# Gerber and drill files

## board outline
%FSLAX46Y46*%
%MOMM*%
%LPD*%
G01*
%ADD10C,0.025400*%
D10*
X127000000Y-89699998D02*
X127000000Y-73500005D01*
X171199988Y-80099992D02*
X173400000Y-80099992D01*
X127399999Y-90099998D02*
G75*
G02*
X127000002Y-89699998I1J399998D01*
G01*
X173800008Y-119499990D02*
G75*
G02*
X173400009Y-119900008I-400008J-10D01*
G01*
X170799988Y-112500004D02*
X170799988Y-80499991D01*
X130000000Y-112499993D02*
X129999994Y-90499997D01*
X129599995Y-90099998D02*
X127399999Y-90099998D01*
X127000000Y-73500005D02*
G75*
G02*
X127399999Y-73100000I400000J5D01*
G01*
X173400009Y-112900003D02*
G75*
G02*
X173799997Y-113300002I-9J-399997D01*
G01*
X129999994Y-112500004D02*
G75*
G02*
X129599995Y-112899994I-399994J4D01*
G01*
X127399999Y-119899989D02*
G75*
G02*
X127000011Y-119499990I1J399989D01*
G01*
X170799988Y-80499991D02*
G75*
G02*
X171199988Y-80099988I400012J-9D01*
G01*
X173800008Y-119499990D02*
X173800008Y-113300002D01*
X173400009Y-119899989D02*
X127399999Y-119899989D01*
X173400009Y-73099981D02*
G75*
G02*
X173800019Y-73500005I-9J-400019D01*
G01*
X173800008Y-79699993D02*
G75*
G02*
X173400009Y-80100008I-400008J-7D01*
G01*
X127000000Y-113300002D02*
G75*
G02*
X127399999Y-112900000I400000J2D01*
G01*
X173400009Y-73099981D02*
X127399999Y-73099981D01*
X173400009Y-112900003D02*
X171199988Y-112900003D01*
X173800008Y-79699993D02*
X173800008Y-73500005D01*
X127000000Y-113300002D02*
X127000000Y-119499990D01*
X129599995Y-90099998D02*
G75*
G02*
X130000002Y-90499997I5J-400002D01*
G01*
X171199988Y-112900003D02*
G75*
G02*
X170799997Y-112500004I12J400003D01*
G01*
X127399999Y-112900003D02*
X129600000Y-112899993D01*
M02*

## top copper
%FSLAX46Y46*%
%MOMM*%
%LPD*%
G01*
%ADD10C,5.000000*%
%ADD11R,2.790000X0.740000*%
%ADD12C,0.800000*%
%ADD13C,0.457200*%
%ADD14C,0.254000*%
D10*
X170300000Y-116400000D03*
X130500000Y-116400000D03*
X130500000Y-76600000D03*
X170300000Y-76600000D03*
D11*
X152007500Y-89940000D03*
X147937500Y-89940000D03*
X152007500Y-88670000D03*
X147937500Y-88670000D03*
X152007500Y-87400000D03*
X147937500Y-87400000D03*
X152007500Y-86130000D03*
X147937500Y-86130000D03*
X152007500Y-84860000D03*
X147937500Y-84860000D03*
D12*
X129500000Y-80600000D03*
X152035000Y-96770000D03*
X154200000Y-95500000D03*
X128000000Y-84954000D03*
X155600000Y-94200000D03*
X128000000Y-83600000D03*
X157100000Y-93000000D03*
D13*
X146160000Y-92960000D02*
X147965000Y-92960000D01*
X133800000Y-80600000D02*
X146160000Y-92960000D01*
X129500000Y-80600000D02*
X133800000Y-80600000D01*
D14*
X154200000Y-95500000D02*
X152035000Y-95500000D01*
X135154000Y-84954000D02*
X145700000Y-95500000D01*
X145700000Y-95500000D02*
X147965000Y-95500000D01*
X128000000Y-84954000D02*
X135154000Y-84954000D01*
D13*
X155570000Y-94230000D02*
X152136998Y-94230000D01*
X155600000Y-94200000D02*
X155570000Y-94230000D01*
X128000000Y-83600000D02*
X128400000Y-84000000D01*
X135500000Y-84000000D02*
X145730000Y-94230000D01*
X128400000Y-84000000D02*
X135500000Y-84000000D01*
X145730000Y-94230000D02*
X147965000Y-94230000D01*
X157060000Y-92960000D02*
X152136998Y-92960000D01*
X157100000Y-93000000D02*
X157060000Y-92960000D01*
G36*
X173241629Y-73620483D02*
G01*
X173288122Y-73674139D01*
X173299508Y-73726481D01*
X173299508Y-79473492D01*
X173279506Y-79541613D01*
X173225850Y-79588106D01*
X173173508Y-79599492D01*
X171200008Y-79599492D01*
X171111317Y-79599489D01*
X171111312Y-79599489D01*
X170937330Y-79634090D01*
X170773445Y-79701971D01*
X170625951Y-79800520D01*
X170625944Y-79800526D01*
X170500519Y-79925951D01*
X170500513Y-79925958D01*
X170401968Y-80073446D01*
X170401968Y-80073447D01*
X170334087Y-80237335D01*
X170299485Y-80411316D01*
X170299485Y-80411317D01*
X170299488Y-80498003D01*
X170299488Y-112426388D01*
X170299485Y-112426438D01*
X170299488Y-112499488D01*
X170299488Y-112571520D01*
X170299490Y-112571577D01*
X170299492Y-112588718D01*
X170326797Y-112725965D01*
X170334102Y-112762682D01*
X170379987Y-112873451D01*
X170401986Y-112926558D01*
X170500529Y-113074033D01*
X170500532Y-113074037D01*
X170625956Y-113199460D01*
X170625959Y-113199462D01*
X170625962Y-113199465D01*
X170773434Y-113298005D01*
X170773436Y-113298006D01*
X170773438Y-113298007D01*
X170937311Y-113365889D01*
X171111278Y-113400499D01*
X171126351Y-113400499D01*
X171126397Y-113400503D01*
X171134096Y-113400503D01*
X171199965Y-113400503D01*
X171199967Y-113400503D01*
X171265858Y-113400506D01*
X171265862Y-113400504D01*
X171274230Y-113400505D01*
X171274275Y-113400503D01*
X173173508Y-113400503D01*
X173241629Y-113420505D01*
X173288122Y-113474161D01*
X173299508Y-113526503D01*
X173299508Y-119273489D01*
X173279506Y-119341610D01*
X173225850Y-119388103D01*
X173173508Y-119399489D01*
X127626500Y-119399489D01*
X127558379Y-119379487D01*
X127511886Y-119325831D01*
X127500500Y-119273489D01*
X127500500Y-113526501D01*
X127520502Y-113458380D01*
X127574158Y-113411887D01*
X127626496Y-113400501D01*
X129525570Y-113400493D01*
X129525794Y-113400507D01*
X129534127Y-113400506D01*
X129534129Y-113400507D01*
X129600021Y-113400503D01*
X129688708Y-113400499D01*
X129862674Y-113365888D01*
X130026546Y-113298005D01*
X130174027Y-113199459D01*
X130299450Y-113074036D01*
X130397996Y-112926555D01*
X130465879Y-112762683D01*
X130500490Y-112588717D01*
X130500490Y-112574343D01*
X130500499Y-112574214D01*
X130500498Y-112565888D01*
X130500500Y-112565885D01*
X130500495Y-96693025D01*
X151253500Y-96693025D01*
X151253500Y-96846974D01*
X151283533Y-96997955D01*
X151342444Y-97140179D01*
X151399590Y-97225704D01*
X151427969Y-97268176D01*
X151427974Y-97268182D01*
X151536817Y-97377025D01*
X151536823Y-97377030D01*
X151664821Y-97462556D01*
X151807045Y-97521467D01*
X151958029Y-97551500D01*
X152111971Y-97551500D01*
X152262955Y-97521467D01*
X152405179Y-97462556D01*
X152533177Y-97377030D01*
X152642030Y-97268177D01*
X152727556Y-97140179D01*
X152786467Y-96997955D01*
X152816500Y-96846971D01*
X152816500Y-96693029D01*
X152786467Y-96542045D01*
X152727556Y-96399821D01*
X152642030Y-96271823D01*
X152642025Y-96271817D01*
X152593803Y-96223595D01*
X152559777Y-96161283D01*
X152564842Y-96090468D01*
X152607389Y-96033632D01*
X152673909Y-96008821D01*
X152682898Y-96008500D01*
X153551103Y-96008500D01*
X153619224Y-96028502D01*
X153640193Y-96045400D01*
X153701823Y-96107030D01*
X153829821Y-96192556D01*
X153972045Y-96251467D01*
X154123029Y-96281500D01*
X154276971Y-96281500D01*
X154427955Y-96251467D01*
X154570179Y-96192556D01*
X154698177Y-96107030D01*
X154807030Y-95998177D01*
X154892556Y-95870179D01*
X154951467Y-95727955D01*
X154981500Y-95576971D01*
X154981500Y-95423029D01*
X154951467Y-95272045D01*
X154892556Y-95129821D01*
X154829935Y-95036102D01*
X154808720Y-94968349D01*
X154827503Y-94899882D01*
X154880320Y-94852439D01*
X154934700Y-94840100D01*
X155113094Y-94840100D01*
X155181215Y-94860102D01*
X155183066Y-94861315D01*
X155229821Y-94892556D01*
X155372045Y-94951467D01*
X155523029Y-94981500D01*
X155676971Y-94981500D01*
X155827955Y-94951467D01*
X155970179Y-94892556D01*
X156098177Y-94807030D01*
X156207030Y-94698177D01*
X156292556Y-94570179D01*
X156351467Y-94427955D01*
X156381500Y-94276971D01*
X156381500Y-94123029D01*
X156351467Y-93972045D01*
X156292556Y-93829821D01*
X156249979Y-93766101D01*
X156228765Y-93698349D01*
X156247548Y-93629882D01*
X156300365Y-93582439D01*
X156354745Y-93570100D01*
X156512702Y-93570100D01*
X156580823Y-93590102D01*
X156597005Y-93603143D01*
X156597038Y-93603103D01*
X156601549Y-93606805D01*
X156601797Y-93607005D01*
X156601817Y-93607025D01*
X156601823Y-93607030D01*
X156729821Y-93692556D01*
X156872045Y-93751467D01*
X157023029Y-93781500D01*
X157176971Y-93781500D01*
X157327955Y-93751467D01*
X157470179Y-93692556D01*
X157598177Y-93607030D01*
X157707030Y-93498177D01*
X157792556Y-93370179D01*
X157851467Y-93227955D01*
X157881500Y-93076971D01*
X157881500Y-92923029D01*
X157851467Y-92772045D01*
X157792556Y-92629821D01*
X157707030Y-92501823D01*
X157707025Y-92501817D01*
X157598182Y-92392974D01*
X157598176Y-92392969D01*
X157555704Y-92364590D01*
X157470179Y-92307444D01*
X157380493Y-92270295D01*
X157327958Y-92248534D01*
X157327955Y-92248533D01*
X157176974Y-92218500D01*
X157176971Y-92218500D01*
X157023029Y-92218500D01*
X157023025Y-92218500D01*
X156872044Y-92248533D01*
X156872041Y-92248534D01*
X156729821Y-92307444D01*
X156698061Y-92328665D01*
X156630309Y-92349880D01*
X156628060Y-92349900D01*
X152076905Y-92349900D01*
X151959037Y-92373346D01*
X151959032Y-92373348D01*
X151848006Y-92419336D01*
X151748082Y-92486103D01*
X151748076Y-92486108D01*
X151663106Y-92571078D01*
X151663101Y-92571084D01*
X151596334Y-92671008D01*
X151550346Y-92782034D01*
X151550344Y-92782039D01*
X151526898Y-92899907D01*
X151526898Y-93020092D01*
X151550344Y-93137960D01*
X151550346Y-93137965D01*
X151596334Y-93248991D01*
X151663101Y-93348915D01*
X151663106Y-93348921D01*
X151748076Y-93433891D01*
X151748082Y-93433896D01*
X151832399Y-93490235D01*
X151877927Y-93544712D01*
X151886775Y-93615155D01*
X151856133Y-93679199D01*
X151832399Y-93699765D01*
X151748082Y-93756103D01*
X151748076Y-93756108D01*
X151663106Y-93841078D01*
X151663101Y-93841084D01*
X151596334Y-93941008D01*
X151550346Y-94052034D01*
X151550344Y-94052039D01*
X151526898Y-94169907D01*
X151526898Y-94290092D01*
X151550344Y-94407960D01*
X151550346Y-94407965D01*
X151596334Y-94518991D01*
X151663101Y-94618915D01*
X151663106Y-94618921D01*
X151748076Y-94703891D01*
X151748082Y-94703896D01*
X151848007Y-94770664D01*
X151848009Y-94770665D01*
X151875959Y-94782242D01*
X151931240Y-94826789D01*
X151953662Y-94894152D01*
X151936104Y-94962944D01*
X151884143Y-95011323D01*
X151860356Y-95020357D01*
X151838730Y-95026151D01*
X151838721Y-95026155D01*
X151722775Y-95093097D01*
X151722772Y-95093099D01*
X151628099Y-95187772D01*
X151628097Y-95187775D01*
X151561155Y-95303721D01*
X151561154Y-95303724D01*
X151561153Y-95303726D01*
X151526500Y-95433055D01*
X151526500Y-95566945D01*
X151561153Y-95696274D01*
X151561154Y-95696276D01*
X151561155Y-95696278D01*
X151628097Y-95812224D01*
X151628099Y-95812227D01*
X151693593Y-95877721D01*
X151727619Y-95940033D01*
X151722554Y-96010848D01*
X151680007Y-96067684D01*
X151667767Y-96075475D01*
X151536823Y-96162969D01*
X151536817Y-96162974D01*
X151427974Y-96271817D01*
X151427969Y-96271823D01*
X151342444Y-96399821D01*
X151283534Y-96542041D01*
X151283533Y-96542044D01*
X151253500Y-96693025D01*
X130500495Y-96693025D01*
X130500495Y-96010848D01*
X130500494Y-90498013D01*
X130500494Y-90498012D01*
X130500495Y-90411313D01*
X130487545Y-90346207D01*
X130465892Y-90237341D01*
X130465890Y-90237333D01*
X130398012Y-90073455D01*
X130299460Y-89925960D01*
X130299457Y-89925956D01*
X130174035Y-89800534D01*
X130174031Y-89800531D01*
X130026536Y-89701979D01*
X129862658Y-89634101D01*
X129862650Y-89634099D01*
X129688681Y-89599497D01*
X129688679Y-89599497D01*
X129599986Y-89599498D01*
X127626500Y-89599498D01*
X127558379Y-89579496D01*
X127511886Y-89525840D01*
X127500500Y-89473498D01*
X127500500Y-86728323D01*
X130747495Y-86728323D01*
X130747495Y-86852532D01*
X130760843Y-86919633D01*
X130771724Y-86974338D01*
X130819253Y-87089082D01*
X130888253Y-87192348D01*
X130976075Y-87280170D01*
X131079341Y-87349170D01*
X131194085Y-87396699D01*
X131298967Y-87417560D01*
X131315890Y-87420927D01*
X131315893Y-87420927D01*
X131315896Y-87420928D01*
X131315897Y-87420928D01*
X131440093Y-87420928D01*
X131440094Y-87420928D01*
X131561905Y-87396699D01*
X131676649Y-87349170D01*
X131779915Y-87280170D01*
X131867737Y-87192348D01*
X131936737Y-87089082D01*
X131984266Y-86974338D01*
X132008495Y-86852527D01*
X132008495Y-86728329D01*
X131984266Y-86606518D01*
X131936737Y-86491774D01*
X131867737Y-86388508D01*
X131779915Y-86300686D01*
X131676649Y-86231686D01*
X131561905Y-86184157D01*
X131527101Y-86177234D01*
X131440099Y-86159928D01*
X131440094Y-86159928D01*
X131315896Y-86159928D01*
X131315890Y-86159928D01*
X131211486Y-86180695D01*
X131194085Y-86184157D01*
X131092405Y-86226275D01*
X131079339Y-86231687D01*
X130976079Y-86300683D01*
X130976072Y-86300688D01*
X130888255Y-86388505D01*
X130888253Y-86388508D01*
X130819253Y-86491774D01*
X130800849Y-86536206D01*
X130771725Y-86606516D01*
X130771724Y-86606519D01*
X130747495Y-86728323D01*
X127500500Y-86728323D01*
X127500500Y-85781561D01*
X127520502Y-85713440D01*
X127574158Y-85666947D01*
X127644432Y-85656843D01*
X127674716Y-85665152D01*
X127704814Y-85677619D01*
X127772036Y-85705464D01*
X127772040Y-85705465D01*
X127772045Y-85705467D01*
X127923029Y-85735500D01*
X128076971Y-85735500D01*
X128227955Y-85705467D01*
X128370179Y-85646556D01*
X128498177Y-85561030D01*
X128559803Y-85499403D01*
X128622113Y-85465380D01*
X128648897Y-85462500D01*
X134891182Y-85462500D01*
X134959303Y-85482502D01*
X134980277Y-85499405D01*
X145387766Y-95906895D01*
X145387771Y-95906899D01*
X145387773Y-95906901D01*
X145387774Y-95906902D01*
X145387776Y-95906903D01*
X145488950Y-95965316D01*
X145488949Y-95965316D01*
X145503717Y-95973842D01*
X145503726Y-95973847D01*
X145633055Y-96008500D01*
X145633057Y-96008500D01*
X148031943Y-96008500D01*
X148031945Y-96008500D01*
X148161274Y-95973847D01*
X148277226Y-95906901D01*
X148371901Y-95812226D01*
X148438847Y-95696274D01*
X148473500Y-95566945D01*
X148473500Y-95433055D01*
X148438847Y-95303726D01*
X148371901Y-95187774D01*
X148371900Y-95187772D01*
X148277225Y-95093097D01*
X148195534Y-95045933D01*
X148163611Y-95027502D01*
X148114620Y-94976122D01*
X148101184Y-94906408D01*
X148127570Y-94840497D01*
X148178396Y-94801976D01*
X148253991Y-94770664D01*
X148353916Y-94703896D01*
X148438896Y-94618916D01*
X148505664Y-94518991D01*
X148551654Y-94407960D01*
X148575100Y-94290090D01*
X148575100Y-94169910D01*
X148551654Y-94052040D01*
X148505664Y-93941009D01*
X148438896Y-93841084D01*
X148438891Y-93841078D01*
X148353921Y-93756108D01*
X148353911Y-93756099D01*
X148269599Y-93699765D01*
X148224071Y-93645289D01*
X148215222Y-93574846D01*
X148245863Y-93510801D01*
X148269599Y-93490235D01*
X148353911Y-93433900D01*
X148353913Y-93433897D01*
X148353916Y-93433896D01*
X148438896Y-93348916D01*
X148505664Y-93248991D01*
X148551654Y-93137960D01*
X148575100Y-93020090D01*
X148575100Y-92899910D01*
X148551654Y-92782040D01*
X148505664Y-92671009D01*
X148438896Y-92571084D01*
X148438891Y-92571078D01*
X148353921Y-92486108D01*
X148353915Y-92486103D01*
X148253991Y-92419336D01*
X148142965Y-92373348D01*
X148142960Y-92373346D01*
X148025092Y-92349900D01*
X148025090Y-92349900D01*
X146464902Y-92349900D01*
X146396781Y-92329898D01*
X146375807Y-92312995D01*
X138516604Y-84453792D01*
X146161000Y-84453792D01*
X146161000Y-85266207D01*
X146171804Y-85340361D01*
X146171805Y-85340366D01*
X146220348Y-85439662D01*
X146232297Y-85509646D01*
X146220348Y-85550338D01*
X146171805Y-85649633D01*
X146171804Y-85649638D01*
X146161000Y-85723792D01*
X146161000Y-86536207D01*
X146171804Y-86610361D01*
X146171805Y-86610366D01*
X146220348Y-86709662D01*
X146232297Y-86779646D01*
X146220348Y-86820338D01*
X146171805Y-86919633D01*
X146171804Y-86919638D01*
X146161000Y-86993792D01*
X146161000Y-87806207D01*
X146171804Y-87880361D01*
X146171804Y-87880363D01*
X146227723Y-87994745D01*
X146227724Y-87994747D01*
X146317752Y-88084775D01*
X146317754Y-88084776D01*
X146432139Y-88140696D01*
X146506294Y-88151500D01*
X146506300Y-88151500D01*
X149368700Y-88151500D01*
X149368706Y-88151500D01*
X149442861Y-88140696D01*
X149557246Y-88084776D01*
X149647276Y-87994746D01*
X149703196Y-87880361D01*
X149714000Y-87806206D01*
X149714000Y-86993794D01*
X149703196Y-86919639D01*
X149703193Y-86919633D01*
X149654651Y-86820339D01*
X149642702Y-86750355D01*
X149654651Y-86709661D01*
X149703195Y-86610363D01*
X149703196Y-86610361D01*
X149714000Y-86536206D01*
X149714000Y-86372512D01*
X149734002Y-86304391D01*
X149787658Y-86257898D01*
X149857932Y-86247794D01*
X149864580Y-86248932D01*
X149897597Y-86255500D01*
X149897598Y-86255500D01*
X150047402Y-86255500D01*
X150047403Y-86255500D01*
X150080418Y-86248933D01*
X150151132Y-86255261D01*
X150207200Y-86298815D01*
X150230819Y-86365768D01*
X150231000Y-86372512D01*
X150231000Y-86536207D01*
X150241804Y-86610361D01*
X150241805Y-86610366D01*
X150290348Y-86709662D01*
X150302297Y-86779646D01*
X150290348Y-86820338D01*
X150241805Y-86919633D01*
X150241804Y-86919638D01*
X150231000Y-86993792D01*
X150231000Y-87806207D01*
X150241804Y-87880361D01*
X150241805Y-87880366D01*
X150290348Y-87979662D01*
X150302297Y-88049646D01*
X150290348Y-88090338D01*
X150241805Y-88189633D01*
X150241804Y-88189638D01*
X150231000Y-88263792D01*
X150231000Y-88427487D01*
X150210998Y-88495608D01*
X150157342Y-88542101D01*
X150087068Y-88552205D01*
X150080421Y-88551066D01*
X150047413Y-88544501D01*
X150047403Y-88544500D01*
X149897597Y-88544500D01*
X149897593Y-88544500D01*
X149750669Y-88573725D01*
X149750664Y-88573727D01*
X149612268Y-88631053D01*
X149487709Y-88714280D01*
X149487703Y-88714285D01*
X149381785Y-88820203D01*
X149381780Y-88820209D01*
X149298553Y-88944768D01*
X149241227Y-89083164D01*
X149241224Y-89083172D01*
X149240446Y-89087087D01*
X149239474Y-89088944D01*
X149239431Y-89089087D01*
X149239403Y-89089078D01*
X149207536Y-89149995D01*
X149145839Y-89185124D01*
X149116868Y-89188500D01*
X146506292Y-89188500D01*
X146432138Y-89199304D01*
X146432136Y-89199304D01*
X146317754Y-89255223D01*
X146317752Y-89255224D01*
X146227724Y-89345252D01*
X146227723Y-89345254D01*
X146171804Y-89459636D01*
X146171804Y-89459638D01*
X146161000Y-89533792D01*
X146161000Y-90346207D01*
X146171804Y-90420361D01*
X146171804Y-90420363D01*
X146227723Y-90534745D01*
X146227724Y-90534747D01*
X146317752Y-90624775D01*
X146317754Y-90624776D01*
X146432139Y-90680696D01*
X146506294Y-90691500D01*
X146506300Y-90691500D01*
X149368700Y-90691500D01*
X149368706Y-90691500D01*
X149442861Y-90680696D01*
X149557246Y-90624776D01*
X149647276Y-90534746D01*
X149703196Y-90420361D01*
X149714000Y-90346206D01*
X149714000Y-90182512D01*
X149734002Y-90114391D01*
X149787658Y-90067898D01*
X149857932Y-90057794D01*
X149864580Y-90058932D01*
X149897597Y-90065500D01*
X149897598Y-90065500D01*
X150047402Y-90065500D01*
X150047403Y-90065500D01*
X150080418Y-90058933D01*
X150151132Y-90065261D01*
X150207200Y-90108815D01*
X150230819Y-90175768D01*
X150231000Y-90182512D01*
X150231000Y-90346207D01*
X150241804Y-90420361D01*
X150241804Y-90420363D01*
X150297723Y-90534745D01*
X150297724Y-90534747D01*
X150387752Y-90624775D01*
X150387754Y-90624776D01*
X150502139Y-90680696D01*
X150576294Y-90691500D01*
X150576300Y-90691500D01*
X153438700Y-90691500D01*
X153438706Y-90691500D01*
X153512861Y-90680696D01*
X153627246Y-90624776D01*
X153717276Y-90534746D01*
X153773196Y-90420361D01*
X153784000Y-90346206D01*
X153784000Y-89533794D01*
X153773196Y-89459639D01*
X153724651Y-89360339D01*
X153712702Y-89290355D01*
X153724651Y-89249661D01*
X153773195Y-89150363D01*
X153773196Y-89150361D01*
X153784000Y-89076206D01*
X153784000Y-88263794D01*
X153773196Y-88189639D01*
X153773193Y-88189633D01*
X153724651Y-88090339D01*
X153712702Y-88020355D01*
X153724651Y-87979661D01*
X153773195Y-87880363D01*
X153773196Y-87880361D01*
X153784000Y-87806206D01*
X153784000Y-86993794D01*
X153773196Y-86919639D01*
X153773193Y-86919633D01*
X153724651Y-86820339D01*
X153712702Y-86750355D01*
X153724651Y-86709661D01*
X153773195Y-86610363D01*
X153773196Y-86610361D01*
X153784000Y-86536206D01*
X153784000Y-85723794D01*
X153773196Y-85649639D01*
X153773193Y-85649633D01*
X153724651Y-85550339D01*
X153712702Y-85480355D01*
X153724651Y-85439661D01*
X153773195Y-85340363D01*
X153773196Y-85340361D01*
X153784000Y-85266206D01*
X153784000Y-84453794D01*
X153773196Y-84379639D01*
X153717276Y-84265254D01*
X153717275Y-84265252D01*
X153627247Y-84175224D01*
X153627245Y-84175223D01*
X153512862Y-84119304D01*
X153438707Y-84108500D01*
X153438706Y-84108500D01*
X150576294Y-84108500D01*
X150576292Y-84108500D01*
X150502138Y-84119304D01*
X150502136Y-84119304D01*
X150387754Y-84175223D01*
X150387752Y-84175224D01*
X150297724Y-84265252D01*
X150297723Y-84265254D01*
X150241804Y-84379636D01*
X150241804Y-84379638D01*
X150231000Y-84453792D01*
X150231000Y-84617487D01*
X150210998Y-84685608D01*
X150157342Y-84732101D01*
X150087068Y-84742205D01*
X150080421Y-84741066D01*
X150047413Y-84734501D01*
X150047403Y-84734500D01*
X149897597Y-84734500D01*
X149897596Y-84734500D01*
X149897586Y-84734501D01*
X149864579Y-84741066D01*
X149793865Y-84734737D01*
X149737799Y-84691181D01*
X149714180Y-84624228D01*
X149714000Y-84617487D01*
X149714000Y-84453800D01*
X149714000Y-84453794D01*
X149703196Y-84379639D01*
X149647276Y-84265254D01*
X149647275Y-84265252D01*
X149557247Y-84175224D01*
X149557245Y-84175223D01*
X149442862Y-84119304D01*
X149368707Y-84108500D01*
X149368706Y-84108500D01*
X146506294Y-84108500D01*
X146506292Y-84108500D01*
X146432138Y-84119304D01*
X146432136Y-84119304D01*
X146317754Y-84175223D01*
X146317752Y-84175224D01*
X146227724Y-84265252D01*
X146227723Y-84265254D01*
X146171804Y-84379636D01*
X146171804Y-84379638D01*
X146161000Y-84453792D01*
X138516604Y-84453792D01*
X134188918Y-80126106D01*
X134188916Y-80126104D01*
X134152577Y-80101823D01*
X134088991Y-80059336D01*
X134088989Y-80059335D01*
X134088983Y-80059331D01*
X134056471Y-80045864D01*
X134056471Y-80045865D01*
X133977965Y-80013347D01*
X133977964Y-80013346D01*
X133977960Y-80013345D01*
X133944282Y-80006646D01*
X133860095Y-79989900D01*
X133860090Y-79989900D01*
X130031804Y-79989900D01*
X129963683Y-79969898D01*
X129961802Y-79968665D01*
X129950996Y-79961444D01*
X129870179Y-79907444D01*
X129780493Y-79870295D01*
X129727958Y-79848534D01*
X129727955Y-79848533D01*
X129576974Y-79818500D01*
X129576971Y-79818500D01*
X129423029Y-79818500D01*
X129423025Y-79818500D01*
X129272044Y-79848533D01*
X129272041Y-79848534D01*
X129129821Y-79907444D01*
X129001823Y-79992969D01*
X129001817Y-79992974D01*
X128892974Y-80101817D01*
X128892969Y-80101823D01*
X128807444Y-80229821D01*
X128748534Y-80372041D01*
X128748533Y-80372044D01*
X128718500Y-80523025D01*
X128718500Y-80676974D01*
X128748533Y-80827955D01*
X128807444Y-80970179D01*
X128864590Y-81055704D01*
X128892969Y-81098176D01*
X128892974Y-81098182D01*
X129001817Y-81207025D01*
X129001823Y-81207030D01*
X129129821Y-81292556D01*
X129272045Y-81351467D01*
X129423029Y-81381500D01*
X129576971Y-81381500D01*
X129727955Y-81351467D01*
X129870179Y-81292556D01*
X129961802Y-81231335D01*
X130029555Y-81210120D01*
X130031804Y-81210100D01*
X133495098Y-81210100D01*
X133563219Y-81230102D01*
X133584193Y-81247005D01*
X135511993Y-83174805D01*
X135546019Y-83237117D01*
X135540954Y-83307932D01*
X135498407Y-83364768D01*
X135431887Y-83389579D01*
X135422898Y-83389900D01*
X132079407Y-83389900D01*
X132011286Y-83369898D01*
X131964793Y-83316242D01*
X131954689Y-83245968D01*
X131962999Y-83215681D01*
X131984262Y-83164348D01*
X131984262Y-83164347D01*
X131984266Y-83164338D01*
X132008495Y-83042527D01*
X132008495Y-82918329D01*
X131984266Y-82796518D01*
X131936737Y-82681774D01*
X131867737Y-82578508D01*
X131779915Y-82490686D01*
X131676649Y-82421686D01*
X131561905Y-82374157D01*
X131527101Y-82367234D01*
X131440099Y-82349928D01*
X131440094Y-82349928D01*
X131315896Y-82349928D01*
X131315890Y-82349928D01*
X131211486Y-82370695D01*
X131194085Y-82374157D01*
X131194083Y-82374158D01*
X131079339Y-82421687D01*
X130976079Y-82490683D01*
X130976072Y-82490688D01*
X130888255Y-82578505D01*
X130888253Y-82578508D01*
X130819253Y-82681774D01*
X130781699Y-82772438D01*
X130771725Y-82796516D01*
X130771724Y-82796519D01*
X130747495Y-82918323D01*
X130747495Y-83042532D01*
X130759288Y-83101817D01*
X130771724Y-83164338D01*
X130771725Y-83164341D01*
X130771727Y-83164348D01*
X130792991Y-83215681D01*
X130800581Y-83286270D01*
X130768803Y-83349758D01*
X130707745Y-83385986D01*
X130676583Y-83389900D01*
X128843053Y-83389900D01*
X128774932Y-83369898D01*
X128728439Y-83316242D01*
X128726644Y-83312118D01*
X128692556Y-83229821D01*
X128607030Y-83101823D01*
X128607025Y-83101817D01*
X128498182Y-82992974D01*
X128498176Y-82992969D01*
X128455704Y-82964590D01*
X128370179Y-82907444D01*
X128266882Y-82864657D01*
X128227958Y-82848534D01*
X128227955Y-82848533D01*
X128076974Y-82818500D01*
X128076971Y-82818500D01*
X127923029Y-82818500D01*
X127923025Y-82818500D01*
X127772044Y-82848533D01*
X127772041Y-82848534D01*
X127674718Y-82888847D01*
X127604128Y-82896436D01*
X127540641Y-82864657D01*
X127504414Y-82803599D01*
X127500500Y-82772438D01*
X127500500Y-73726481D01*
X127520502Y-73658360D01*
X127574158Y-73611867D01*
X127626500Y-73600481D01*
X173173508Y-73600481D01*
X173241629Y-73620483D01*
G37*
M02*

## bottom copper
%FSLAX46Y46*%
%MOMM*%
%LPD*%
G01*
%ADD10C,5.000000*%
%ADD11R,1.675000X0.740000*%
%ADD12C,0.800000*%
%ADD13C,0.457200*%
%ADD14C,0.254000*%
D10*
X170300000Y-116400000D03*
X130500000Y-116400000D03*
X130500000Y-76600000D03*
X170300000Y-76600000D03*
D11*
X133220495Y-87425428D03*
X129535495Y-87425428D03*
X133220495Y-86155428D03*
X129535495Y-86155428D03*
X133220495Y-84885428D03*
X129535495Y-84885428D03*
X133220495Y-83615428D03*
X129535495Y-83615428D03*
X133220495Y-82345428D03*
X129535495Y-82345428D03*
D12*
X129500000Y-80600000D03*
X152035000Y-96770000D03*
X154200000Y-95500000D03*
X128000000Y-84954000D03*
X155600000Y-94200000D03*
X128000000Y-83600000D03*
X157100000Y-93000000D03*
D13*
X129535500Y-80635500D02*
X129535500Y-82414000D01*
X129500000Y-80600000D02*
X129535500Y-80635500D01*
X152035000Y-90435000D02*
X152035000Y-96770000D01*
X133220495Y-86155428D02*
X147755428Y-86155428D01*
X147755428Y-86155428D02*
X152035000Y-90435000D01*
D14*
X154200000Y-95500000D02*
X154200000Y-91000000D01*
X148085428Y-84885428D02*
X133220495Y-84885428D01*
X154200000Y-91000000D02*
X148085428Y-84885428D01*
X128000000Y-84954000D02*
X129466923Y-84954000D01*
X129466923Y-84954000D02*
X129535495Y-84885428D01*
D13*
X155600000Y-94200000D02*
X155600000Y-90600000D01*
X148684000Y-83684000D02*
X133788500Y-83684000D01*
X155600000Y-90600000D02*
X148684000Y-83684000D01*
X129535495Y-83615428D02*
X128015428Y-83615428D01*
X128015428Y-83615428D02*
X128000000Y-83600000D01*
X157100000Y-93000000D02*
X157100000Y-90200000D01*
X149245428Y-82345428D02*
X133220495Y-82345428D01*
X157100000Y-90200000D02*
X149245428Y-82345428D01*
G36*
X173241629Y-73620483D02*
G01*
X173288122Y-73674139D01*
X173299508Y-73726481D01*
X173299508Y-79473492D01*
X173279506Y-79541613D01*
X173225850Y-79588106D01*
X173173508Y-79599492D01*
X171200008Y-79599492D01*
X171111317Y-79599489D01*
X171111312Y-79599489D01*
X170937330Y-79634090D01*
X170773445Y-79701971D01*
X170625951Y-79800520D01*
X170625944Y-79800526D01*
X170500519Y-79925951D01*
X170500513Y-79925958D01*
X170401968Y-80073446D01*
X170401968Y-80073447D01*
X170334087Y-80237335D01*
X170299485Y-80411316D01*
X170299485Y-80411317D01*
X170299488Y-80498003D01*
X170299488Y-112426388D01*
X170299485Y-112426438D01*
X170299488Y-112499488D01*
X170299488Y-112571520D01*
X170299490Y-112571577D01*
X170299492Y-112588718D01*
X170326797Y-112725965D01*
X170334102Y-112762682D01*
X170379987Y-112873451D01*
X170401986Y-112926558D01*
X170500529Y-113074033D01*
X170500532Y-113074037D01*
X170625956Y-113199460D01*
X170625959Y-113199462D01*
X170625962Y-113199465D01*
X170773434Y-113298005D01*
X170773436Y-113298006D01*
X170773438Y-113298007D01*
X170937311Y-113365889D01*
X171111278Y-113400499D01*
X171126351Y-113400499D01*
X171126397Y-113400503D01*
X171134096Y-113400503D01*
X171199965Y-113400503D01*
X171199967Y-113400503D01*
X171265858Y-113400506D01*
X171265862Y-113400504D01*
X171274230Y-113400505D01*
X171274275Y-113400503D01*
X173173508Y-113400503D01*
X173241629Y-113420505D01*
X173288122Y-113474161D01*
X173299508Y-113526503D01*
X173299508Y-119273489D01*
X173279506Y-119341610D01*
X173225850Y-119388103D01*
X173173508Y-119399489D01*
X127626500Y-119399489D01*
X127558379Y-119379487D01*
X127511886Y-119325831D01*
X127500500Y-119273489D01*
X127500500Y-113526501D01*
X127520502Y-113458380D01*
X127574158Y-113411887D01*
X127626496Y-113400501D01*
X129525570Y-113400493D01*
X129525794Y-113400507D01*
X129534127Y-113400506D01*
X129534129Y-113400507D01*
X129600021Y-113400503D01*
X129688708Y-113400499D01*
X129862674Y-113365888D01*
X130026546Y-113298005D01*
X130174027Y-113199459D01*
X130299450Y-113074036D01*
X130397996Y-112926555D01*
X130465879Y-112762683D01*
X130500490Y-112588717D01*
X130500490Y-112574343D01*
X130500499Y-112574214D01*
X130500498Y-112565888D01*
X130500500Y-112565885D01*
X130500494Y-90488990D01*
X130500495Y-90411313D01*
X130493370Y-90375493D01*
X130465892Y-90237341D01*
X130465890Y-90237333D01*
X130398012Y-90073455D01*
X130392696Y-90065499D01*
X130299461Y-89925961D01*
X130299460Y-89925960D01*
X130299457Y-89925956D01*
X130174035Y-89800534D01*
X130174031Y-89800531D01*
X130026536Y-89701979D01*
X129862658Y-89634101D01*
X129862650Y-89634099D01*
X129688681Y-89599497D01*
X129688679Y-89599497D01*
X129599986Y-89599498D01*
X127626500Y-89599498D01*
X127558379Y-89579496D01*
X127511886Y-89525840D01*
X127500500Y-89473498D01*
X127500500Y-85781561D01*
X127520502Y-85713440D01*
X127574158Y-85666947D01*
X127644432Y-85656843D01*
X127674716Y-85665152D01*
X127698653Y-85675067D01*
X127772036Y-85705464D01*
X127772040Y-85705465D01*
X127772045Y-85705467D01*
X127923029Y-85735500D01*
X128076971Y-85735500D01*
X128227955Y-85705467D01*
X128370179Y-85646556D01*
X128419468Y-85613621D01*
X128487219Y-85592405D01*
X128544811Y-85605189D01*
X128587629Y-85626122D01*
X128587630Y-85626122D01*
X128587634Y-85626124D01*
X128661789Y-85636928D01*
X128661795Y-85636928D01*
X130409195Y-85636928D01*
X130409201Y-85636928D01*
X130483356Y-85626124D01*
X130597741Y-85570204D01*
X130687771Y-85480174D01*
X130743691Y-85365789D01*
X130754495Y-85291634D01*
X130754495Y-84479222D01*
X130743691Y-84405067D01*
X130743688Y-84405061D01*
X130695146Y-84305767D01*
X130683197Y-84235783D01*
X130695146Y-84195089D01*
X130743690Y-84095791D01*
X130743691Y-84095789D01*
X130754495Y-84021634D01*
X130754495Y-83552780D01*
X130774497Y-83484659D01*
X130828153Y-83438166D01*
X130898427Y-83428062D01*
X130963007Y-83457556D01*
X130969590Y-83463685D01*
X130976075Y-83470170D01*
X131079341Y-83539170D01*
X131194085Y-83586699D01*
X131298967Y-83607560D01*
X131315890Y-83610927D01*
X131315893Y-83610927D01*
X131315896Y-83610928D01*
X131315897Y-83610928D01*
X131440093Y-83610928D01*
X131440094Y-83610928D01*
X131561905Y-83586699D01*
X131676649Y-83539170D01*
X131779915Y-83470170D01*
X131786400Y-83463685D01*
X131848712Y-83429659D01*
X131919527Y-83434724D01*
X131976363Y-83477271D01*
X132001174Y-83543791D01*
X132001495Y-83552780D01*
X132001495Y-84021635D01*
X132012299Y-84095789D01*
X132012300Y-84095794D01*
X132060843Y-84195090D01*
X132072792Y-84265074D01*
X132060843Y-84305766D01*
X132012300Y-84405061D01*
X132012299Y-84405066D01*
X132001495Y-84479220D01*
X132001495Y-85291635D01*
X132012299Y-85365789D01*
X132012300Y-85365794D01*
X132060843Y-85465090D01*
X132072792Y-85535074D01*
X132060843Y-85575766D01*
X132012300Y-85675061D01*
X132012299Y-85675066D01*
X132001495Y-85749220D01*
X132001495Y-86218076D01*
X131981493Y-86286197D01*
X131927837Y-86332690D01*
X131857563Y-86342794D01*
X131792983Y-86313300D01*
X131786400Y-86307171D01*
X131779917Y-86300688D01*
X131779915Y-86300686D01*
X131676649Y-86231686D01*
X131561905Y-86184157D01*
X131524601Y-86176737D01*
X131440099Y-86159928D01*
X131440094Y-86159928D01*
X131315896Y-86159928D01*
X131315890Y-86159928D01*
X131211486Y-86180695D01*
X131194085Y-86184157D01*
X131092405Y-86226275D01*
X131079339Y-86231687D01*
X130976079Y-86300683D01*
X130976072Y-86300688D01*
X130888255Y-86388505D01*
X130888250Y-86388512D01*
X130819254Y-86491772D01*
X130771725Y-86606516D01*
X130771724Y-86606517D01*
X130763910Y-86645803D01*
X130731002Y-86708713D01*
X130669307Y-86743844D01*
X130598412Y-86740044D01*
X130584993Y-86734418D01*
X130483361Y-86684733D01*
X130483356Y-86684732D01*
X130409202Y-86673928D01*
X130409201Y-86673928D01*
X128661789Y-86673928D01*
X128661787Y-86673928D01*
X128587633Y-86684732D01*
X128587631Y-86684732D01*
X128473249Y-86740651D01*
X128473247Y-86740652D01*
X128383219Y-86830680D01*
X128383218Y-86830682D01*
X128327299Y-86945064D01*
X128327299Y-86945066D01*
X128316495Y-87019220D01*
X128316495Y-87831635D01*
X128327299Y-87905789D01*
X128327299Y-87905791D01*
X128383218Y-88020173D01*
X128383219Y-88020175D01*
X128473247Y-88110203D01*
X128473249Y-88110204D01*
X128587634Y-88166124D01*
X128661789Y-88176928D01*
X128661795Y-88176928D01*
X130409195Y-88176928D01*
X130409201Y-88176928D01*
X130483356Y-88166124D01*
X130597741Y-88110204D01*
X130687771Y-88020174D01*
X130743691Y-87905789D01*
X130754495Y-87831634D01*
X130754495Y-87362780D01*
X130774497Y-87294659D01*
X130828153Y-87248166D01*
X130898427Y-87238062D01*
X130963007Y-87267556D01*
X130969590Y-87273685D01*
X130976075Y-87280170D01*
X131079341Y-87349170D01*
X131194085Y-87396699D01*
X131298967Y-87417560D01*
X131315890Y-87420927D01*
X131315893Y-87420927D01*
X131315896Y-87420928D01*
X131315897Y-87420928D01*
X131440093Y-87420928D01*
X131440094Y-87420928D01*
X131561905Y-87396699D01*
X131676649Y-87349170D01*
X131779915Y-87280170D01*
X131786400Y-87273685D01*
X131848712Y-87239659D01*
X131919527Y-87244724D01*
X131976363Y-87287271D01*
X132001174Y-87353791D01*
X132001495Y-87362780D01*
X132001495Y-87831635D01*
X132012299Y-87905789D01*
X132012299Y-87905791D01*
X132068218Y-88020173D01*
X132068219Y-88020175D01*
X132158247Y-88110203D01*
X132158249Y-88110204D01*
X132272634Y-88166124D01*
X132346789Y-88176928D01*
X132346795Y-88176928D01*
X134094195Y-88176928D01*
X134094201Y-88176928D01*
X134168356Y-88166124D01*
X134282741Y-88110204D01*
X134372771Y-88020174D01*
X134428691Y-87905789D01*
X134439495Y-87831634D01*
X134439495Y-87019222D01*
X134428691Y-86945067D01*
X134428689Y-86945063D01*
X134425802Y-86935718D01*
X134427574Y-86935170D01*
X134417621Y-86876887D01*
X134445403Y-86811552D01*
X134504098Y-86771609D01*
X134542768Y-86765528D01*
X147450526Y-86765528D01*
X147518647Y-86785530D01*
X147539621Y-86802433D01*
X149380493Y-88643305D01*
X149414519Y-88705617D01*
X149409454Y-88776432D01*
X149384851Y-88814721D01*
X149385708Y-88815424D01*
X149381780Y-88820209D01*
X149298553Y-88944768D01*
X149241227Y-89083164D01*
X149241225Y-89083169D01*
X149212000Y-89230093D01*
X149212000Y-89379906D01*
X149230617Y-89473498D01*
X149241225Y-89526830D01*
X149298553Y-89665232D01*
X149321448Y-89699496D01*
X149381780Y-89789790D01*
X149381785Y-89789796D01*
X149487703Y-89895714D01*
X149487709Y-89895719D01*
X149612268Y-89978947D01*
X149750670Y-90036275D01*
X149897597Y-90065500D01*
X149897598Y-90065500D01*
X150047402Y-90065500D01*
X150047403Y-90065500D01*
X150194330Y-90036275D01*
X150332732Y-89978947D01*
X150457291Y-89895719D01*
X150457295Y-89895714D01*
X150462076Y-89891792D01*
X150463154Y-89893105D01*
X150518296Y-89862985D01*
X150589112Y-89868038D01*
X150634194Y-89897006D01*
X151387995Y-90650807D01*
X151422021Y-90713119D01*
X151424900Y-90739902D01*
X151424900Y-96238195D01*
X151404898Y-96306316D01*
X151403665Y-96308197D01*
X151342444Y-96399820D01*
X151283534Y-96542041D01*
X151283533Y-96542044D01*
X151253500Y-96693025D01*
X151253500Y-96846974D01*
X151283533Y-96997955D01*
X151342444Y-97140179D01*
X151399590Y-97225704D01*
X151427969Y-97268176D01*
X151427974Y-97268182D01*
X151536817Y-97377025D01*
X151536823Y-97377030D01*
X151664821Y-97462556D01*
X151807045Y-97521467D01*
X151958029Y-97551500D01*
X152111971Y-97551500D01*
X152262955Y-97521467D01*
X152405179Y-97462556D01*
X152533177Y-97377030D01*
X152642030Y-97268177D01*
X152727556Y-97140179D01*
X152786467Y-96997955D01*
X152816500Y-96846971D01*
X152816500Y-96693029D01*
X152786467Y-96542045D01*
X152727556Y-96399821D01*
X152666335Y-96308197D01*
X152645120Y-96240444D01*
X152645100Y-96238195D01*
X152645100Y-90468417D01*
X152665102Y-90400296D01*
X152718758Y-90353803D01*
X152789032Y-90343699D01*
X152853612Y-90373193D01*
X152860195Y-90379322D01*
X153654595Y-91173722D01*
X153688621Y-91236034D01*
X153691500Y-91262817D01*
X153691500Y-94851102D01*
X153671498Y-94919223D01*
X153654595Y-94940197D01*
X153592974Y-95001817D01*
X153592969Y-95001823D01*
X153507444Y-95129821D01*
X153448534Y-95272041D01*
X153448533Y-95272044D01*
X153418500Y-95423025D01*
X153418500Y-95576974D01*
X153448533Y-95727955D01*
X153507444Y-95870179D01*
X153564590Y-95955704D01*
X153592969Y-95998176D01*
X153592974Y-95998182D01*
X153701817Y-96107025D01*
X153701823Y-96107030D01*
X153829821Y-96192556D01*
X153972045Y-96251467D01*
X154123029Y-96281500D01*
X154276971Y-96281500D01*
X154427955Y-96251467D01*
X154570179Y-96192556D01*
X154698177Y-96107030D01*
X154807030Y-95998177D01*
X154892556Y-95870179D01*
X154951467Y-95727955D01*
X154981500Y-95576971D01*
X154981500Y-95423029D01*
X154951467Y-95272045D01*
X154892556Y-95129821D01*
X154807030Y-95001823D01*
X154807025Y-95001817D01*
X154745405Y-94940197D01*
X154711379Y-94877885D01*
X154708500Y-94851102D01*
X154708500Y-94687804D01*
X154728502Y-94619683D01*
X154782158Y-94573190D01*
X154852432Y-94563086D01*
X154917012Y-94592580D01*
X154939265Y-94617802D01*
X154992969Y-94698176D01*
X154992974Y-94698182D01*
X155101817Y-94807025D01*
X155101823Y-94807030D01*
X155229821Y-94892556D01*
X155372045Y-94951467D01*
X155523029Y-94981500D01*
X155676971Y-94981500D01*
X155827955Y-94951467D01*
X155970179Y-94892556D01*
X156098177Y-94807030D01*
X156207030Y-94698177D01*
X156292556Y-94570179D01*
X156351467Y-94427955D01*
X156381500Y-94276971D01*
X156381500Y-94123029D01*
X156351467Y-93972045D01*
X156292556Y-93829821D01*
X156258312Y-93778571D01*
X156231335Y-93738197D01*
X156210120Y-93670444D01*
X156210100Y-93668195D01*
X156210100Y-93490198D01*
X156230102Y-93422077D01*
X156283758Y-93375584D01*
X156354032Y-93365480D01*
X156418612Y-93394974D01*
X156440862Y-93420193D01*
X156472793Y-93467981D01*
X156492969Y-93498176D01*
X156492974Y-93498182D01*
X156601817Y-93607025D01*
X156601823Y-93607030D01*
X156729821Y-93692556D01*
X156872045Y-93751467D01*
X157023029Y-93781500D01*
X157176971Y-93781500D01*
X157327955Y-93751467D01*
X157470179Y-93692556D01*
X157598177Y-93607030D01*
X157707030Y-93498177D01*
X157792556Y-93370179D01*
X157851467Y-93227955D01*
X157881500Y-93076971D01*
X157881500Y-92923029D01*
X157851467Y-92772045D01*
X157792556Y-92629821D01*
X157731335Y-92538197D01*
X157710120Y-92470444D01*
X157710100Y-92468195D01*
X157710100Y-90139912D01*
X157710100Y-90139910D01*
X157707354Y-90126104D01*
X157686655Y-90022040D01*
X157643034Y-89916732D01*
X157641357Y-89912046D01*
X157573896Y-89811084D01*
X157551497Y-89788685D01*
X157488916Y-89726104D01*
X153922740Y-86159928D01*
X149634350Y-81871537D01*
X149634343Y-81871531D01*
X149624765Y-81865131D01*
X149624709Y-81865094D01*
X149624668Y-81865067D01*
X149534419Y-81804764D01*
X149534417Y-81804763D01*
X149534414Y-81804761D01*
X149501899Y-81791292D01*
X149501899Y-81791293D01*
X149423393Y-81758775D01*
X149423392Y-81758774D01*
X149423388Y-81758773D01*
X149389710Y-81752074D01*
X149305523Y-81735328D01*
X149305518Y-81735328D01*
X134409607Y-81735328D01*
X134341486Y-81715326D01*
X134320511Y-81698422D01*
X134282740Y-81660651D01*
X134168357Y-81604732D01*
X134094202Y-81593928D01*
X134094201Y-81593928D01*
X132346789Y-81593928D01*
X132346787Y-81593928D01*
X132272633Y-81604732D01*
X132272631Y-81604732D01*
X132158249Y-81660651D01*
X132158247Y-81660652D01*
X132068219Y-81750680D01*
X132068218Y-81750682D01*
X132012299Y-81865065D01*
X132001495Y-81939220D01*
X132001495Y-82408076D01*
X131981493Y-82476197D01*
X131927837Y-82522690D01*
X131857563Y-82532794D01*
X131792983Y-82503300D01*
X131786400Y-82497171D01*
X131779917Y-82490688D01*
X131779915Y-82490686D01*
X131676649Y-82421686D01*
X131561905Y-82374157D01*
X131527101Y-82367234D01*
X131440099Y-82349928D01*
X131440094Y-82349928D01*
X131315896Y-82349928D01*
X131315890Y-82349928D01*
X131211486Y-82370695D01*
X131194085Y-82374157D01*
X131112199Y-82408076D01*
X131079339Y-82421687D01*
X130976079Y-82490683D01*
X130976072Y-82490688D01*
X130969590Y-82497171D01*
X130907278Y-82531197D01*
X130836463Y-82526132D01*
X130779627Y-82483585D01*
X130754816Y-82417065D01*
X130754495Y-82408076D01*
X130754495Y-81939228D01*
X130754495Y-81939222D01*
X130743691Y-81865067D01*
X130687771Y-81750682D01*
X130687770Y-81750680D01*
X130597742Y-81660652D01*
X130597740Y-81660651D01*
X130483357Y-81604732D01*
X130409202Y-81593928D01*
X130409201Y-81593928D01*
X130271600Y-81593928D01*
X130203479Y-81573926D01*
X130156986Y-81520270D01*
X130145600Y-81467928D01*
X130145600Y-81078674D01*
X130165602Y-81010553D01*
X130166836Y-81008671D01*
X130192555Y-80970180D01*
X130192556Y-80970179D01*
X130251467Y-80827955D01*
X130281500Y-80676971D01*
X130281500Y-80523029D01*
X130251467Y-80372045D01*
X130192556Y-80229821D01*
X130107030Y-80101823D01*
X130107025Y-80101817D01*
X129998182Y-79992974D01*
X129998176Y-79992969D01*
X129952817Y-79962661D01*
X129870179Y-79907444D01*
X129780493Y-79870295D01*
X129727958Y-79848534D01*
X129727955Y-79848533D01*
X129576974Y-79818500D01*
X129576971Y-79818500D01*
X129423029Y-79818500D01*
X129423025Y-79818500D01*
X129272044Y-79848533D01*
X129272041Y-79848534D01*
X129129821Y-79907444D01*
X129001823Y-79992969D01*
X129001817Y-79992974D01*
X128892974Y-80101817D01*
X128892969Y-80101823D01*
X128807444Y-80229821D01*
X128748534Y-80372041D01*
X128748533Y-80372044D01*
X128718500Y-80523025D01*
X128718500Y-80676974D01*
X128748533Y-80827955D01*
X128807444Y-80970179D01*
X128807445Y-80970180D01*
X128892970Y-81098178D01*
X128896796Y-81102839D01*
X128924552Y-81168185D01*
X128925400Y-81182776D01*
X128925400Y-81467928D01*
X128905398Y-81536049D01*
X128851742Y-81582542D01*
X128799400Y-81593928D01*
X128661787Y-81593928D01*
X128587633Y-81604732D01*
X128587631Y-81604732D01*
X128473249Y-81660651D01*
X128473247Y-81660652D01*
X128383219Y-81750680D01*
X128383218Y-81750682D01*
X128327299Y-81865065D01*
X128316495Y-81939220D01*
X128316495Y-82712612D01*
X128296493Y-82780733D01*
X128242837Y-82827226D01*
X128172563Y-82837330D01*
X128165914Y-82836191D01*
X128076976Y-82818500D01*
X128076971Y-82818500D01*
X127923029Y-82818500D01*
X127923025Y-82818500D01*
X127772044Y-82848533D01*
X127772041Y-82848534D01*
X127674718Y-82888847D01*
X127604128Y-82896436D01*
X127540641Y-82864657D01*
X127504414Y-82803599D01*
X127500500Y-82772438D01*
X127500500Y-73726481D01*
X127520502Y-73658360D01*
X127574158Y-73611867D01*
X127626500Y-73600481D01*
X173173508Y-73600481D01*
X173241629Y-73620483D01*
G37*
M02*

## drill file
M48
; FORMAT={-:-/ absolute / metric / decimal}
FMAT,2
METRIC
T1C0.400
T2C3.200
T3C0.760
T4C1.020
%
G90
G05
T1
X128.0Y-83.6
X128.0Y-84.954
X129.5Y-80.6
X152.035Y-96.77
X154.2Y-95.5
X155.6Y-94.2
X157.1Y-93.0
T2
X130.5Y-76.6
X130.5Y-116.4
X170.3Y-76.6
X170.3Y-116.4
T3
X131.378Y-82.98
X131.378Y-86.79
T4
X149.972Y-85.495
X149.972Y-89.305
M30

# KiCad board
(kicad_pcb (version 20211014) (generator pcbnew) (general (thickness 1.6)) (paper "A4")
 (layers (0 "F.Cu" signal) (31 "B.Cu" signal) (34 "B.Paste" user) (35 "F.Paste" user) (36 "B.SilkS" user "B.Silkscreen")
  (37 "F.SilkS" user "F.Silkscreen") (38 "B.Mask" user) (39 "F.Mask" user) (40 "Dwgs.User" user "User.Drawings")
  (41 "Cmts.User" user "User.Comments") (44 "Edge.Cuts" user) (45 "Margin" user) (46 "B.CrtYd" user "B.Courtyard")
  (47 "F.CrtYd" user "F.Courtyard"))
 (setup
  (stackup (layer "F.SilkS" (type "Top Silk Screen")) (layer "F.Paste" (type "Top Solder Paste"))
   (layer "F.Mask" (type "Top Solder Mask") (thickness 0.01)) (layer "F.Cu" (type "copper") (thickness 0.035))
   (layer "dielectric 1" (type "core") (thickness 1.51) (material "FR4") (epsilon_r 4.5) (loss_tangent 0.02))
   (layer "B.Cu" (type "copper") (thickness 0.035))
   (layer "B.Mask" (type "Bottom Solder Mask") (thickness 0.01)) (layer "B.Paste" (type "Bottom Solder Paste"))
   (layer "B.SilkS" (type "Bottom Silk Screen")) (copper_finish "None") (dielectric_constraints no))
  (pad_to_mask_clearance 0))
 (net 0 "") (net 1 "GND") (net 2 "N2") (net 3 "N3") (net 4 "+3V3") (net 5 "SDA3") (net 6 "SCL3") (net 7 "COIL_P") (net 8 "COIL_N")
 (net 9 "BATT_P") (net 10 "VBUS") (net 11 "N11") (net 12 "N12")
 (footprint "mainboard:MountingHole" (layer "F.Cu") (at 170.3 116.4 -90)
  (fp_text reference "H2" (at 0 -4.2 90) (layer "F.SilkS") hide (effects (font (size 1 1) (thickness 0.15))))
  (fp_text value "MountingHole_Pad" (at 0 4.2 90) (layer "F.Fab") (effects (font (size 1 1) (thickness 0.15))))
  (pad "1" thru_hole circle (at 0 0 270) (size 5 5) (drill 3.2) (layers *.Cu *.Mask) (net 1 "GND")))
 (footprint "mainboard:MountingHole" (layer "F.Cu") (at 130.5 116.4 -90)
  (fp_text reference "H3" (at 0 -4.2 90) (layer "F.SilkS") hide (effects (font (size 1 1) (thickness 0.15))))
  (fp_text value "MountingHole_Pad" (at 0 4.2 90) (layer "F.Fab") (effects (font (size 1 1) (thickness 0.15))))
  (pad "1" thru_hole circle (at 0 0 270) (size 5 5) (drill 3.2) (layers *.Cu *.Mask) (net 1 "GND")))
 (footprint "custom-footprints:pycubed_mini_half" (layer "F.Cu") (at 151.251997 75.817212)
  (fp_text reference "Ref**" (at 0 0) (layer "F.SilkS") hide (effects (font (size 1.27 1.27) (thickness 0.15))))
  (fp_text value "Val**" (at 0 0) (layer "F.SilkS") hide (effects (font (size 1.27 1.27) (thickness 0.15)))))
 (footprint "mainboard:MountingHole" (layer "F.Cu") (at 130.5 76.6 -90)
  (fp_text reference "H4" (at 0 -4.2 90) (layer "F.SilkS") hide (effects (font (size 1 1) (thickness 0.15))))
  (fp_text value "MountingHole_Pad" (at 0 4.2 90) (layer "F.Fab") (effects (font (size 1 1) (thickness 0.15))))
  (pad "1" thru_hole circle (at 0 0 270) (size 5 5) (drill 3.2) (layers *.Cu *.Mask) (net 1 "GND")))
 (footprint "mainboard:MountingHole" (layer "F.Cu") (at 170.3 76.6 -90)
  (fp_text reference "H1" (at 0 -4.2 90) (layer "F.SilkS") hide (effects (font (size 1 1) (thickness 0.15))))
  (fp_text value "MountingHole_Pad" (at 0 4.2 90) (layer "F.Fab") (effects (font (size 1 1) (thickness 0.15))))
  (pad "1" thru_hole circle (at 0 0 270) (size 5 5) (drill 3.2) (layers *.Cu *.Mask) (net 1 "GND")))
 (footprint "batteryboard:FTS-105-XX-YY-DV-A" (layer "F.Cu") (at 149.9725 87.4 90)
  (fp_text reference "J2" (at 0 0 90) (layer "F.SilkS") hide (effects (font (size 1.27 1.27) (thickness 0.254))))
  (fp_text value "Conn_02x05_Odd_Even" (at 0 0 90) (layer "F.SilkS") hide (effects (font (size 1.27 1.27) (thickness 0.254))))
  (pad "" np_thru_hole circle (at 1.905 0 90) (size 1.02 1.02) (drill 1.02) (layers *.Cu *.Mask))
  (pad "" np_thru_hole circle (at -1.905 0 90) (size 1.02 1.02) (drill 1.02) (layers *.Cu *.Mask))
  (pad "1" smd rect (at -2.54 2.035 90) (size 0.74 2.79) (layers "F.Cu" "F.Paste" "F.Mask") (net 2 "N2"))
  (pad "2" smd rect (at -2.54 -2.035 90) (size 0.74 2.79) (layers "F.Cu" "F.Paste" "F.Mask") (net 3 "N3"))
  (pad "3" smd rect (at -1.27 2.035 90) (size 0.74 2.79) (layers "F.Cu" "F.Paste" "F.Mask") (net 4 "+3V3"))
  (pad "4" smd rect (at -1.27 -2.035 90) (size 0.74 2.79) (layers "F.Cu" "F.Paste" "F.Mask") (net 1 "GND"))
  (pad "5" smd rect (at 0 2.035 90) (size 0.74 2.79) (layers "F.Cu" "F.Paste" "F.Mask") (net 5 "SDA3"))
  (pad "6" smd rect (at 0 -2.035 90) (size 0.74 2.79) (layers "F.Cu" "F.Paste" "F.Mask") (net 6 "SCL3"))
  (pad "7" smd rect (at 1.27 2.035 90) (size 0.74 2.79) (layers "F.Cu" "F.Paste" "F.Mask") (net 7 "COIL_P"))
  (pad "8" smd rect (at 1.27 -2.035 90) (size 0.74 2.79) (layers "F.Cu" "F.Paste" "F.Mask") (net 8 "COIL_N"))
  (pad "9" smd rect (at 2.54 2.035 90) (size 0.74 2.79) (layers "F.Cu" "F.Paste" "F.Mask") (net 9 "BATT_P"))
  (pad "10" smd rect (at 2.54 -2.035 90) (size 0.74 2.79) (layers "F.Cu" "F.Paste" "F.Mask") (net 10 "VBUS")))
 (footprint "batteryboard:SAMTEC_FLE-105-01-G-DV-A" (layer "B.Cu") (at 131.377995 84.885428 90)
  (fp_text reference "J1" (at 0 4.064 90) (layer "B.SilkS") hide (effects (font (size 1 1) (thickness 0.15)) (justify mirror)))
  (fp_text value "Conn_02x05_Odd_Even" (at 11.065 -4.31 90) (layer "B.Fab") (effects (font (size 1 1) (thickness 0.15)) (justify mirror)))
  (pad "" np_thru_hole circle (at -1.905 0 90) (size 0.76 0.76) (drill 0.76) (layers *.Cu *.Mask))
  (pad "" np_thru_hole circle (at 1.905 0 90) (size 0.76 0.76) (drill 0.76) (layers *.Cu *.Mask))
  (pad "01" smd rect (at -2.54 1.8425 90) (size 0.74 1.675) (layers "B.Cu" "B.Paste" "B.Mask") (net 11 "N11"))
  (pad "02" smd rect (at -2.54 -1.8425 90) (size 0.74 1.675) (layers "B.Cu" "B.Paste" "B.Mask") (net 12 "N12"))
  (pad "03" smd rect (at -1.27 1.8425 90) (size 0.74 1.675) (layers "B.Cu" "B.Paste" "B.Mask") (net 4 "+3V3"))
  (pad "04" smd rect (at -1.27 -1.8425 90) (size 0.74 1.675) (layers "B.Cu" "B.Paste" "B.Mask") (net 1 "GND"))
  (pad "05" smd rect (at 0 1.8425 90) (size 0.74 1.675) (layers "B.Cu" "B.Paste" "B.Mask") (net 5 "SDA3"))
  (pad "06" smd rect (at 0 -1.8425 90) (size 0.74 1.675) (layers "B.Cu" "B.Paste" "B.Mask") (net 6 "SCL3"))
  (pad "07" smd rect (at 1.27 1.8425 90) (size 0.74 1.675) (layers "B.Cu" "B.Paste" "B.Mask") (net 7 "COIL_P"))
  (pad "08" smd rect (at 1.27 -1.8425 90) (size 0.74 1.675) (layers "B.Cu" "B.Paste" "B.Mask") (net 8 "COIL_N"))
  (pad "09" smd rect (at 2.54 1.8425 90) (size 0.74 1.675) (layers "B.Cu" "B.Paste" "B.Mask") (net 9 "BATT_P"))
  (pad "10" smd rect (at 2.54 -1.8425 90) (size 0.74 1.675) (layers "B.Cu" "B.Paste" "B.Mask") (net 10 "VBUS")))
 (gr_line (start 127 89.699998) (end 127 73.500005) (layer "Edge.Cuts") (width 0.0254))
 (gr_line (start 171.199988 80.099992) (end 173.4 80.099992) (layer "Edge.Cuts") (width 0.0254))
 (gr_arc (start 127.399999 90.099998) (mid 127.117156 89.982842) (end 127 89.699998) (layer "Edge.Cuts") (width 0.0254))
 (gr_arc (start 173.800008 119.49999) (mid 173.682852 119.782833) (end 173.400009 119.899989) (layer "Edge.Cuts") (width 0.0254))
 (gr_line (start 170.799988 112.500004) (end 170.799988 80.499991) (layer "Edge.Cuts") (width 0.0254))
 (gr_line (start 130 112.499993) (end 129.999994 90.499997) (layer "Edge.Cuts") (width 0.0254))
 (gr_line (start 129.599995 90.099998) (end 127.399999 90.099998) (layer "Edge.Cuts") (width 0.0254))
 (gr_arc (start 127 73.500005) (mid 127.117155 73.217153) (end 127.399999 73.099981) (layer "Edge.Cuts") (width 0.0254))
 (gr_arc (start 173.400009 112.900003) (mid 173.682845 113.017166) (end 173.800008 113.300002) (layer "Edge.Cuts") (width 0.0254))
 (gr_arc (start 129.999994 112.500004) (mid 129.882831 112.78284) (end 129.599995 112.900003) (layer "Edge.Cuts") (width 0.0254))
 (gr_arc (start 127.399999 119.899989) (mid 127.117158 119.782831) (end 127 119.49999) (layer "Edge.Cuts") (width 0.0254))
 (gr_arc (start 170.799988 80.499991) (mid 170.917141 80.217144) (end 171.199988 80.099992) (layer "Edge.Cuts") (width 0.0254))
 (gr_line (start 173.800008 119.49999) (end 173.800008 113.300002) (layer "Edge.Cuts") (width 0.0254))
 (gr_line (start 173.400009 119.899989) (end 127.399999 119.899989) (layer "Edge.Cuts") (width 0.0254))
 (gr_arc (start 173.400009 73.099981) (mid 173.682859 73.217147) (end 173.800008 73.500005) (layer "Edge.Cuts") (width 0.0254))
 (gr_arc (start 173.800008 79.699993) (mid 173.68285 79.982834) (end 173.400009 80.099992) (layer "Edge.Cuts") (width 0.0254))
 (gr_arc (start 127 113.300002) (mid 127.117153 113.017156) (end 127.399999 112.900003) (layer "Edge.Cuts") (width 0.0254))
 (gr_line (start 173.400009 73.099981) (end 127.399999 73.099981) (layer "Edge.Cuts") (width 0.0254))
 (gr_line (start 173.400009 112.900003) (end 171.199988 112.900003) (layer "Edge.Cuts") (width 0.0254))
 (gr_line (start 173.800008 79.699993) (end 173.800008 73.500005) (layer "Edge.Cuts") (width 0.0254))
 (gr_line (start 127 113.300002) (end 127 119.49999) (layer "Edge.Cuts") (width 0.0254))
 (gr_arc (start 129.599995 90.099998) (mid 129.882839 90.217153) (end 129.999994 90.499997) (layer "Edge.Cuts") (width 0.0254))
 (gr_arc (start 171.199988 112.900003) (mid 170.917151 112.782841) (end 170.799988 112.500004) (layer "Edge.Cuts") (width 0.0254))
 (gr_line (start 127.399999 112.900003) (end 129.6 112.899993) (layer "Edge.Cuts") (width 0.0254))
 (segment (start 146.16 92.96) (end 147.965 92.96) (width 0.4572) (layer "F.Cu") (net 10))
 (segment (start 133.8 80.6) (end 146.16 92.96) (width 0.4572) (layer "F.Cu") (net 10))
 (segment (start 129.5 80.6) (end 133.8 80.6) (width 0.4572) (layer "F.Cu") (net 10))
 (via (at 129.5 80.6) (size 0.8) (drill 0.4) (layers "F.Cu" "B.Cu") (free) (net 10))
 (segment (start 129.5355 80.6355) (end 129.5355 82.414) (width 0.4572) (layer "B.Cu") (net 10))
 (segment (start 129.5 80.6) (end 129.5355 80.6355) (width 0.4572) (layer "B.Cu") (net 10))
 (via (at 152.035 96.77) (size 0.8) (drill 0.4) (layers "F.Cu" "B.Cu") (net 4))
 (segment (start 152.035 90.435) (end 152.035 96.77) (width 0.4572) (layer "B.Cu") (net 4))
 (segment (start 133.220495 86.155428) (end 147.755428 86.155428) (width 0.4572) (layer "B.Cu") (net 4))
 (segment (start 147.755428 86.155428) (end 152.035 90.435) (width 0.4572) (layer "B.Cu") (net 4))
 (segment (start 154.2 95.5) (end 152.035 95.5) (width 0.254) (layer "F.Cu") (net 5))
 (via (at 154.2 95.5) (size 0.8) (drill 0.4) (layers "F.Cu" "B.Cu") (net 5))
 (segment (start 154.2 95.5) (end 154.2 91) (width 0.254) (layer "B.Cu") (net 5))
 (segment (start 148.085428 84.885428) (end 133.220495 84.885428) (width 0.254) (layer "B.Cu") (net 5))
 (segment (start 154.2 91) (end 148.085428 84.885428) (width 0.254) (layer "B.Cu") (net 5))
 (segment (start 135.154 84.954) (end 145.7 95.5) (width 0.254) (layer "F.Cu") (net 6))
 (segment (start 145.7 95.5) (end 147.965 95.5) (width 0.254) (layer "F.Cu") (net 6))
 (segment (start 128 84.954) (end 135.154 84.954) (width 0.254) (layer "F.Cu") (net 6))
 (via (at 128 84.954) (size 0.8) (drill 0.4) (layers "F.Cu" "B.Cu") (free) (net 6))
 (segment (start 128 84.954) (end 129.466923 84.954) (width 0.254) (layer "B.Cu") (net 6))
 (segment (start 129.466923 84.954) (end 129.535495 84.885428) (width 0.254) (layer "B.Cu") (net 6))
 (segment (start 155.57 94.23) (end 152.136998 94.23) (width 0.4572) (layer "F.Cu") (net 7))
 (segment (start 155.6 94.2) (end 155.57 94.23) (width 0.4572) (layer "F.Cu") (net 7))
 (via (at 155.6 94.2) (size 0.8) (drill 0.4) (layers "F.Cu" "B.Cu") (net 7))
 (segment (start 155.6 94.2) (end 155.6 90.6) (width 0.4572) (layer "B.Cu") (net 7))
 (segment (start 148.684 83.684) (end 133.7885 83.684) (width 0.4572) (layer "B.Cu") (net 7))
 (segment (start 155.6 90.6) (end 148.684 83.684) (width 0.4572) (layer "B.Cu") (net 7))
 (segment (start 128 83.6) (end 128.4 84) (width 0.4572) (layer "F.Cu") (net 8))
 (segment (start 135.5 84) (end 145.73 94.23) (width 0.4572) (layer "F.Cu") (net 8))
 (segment (start 128.4 84) (end 135.5 84) (width 0.4572) (layer "F.Cu") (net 8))
 (segment (start 145.73 94.23) (end 147.965 94.23) (width 0.4572) (layer "F.Cu") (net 8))
 (via (at 128 83.6) (size 0.8) (drill 0.4) (layers "F.Cu" "B.Cu") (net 8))
 (segment (start 129.535495 83.615428) (end 128.015428 83.615428) (width 0.4572) (layer "B.Cu") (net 8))
 (segment (start 128.015428 83.615428) (end 128 83.6) (width 0.4572) (layer "B.Cu") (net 8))
 (segment (start 157.06 92.96) (end 152.136998 92.96) (width 0.4572) (layer "F.Cu") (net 9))
 (segment (start 157.1 93) (end 157.06 92.96) (width 0.4572) (layer "F.Cu") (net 9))
 (via (at 157.1 93) (size 0.8) (drill 0.4) (layers "F.Cu" "B.Cu") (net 9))
 (segment (start 157.1 93) (end 157.1 90.2) (width 0.4572) (layer "B.Cu") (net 9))
 (segment (start 149.245428 82.345428) (end 133.220495 82.345428) (width 0.4572) (layer "B.Cu") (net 9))
 (segment (start 157.1 90.2) (end 149.245428 82.345428) (width 0.4572) (layer "B.Cu") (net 9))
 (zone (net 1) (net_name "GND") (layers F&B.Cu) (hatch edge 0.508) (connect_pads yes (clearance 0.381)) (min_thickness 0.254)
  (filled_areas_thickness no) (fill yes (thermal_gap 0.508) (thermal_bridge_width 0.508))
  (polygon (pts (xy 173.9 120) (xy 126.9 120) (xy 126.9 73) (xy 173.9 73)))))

